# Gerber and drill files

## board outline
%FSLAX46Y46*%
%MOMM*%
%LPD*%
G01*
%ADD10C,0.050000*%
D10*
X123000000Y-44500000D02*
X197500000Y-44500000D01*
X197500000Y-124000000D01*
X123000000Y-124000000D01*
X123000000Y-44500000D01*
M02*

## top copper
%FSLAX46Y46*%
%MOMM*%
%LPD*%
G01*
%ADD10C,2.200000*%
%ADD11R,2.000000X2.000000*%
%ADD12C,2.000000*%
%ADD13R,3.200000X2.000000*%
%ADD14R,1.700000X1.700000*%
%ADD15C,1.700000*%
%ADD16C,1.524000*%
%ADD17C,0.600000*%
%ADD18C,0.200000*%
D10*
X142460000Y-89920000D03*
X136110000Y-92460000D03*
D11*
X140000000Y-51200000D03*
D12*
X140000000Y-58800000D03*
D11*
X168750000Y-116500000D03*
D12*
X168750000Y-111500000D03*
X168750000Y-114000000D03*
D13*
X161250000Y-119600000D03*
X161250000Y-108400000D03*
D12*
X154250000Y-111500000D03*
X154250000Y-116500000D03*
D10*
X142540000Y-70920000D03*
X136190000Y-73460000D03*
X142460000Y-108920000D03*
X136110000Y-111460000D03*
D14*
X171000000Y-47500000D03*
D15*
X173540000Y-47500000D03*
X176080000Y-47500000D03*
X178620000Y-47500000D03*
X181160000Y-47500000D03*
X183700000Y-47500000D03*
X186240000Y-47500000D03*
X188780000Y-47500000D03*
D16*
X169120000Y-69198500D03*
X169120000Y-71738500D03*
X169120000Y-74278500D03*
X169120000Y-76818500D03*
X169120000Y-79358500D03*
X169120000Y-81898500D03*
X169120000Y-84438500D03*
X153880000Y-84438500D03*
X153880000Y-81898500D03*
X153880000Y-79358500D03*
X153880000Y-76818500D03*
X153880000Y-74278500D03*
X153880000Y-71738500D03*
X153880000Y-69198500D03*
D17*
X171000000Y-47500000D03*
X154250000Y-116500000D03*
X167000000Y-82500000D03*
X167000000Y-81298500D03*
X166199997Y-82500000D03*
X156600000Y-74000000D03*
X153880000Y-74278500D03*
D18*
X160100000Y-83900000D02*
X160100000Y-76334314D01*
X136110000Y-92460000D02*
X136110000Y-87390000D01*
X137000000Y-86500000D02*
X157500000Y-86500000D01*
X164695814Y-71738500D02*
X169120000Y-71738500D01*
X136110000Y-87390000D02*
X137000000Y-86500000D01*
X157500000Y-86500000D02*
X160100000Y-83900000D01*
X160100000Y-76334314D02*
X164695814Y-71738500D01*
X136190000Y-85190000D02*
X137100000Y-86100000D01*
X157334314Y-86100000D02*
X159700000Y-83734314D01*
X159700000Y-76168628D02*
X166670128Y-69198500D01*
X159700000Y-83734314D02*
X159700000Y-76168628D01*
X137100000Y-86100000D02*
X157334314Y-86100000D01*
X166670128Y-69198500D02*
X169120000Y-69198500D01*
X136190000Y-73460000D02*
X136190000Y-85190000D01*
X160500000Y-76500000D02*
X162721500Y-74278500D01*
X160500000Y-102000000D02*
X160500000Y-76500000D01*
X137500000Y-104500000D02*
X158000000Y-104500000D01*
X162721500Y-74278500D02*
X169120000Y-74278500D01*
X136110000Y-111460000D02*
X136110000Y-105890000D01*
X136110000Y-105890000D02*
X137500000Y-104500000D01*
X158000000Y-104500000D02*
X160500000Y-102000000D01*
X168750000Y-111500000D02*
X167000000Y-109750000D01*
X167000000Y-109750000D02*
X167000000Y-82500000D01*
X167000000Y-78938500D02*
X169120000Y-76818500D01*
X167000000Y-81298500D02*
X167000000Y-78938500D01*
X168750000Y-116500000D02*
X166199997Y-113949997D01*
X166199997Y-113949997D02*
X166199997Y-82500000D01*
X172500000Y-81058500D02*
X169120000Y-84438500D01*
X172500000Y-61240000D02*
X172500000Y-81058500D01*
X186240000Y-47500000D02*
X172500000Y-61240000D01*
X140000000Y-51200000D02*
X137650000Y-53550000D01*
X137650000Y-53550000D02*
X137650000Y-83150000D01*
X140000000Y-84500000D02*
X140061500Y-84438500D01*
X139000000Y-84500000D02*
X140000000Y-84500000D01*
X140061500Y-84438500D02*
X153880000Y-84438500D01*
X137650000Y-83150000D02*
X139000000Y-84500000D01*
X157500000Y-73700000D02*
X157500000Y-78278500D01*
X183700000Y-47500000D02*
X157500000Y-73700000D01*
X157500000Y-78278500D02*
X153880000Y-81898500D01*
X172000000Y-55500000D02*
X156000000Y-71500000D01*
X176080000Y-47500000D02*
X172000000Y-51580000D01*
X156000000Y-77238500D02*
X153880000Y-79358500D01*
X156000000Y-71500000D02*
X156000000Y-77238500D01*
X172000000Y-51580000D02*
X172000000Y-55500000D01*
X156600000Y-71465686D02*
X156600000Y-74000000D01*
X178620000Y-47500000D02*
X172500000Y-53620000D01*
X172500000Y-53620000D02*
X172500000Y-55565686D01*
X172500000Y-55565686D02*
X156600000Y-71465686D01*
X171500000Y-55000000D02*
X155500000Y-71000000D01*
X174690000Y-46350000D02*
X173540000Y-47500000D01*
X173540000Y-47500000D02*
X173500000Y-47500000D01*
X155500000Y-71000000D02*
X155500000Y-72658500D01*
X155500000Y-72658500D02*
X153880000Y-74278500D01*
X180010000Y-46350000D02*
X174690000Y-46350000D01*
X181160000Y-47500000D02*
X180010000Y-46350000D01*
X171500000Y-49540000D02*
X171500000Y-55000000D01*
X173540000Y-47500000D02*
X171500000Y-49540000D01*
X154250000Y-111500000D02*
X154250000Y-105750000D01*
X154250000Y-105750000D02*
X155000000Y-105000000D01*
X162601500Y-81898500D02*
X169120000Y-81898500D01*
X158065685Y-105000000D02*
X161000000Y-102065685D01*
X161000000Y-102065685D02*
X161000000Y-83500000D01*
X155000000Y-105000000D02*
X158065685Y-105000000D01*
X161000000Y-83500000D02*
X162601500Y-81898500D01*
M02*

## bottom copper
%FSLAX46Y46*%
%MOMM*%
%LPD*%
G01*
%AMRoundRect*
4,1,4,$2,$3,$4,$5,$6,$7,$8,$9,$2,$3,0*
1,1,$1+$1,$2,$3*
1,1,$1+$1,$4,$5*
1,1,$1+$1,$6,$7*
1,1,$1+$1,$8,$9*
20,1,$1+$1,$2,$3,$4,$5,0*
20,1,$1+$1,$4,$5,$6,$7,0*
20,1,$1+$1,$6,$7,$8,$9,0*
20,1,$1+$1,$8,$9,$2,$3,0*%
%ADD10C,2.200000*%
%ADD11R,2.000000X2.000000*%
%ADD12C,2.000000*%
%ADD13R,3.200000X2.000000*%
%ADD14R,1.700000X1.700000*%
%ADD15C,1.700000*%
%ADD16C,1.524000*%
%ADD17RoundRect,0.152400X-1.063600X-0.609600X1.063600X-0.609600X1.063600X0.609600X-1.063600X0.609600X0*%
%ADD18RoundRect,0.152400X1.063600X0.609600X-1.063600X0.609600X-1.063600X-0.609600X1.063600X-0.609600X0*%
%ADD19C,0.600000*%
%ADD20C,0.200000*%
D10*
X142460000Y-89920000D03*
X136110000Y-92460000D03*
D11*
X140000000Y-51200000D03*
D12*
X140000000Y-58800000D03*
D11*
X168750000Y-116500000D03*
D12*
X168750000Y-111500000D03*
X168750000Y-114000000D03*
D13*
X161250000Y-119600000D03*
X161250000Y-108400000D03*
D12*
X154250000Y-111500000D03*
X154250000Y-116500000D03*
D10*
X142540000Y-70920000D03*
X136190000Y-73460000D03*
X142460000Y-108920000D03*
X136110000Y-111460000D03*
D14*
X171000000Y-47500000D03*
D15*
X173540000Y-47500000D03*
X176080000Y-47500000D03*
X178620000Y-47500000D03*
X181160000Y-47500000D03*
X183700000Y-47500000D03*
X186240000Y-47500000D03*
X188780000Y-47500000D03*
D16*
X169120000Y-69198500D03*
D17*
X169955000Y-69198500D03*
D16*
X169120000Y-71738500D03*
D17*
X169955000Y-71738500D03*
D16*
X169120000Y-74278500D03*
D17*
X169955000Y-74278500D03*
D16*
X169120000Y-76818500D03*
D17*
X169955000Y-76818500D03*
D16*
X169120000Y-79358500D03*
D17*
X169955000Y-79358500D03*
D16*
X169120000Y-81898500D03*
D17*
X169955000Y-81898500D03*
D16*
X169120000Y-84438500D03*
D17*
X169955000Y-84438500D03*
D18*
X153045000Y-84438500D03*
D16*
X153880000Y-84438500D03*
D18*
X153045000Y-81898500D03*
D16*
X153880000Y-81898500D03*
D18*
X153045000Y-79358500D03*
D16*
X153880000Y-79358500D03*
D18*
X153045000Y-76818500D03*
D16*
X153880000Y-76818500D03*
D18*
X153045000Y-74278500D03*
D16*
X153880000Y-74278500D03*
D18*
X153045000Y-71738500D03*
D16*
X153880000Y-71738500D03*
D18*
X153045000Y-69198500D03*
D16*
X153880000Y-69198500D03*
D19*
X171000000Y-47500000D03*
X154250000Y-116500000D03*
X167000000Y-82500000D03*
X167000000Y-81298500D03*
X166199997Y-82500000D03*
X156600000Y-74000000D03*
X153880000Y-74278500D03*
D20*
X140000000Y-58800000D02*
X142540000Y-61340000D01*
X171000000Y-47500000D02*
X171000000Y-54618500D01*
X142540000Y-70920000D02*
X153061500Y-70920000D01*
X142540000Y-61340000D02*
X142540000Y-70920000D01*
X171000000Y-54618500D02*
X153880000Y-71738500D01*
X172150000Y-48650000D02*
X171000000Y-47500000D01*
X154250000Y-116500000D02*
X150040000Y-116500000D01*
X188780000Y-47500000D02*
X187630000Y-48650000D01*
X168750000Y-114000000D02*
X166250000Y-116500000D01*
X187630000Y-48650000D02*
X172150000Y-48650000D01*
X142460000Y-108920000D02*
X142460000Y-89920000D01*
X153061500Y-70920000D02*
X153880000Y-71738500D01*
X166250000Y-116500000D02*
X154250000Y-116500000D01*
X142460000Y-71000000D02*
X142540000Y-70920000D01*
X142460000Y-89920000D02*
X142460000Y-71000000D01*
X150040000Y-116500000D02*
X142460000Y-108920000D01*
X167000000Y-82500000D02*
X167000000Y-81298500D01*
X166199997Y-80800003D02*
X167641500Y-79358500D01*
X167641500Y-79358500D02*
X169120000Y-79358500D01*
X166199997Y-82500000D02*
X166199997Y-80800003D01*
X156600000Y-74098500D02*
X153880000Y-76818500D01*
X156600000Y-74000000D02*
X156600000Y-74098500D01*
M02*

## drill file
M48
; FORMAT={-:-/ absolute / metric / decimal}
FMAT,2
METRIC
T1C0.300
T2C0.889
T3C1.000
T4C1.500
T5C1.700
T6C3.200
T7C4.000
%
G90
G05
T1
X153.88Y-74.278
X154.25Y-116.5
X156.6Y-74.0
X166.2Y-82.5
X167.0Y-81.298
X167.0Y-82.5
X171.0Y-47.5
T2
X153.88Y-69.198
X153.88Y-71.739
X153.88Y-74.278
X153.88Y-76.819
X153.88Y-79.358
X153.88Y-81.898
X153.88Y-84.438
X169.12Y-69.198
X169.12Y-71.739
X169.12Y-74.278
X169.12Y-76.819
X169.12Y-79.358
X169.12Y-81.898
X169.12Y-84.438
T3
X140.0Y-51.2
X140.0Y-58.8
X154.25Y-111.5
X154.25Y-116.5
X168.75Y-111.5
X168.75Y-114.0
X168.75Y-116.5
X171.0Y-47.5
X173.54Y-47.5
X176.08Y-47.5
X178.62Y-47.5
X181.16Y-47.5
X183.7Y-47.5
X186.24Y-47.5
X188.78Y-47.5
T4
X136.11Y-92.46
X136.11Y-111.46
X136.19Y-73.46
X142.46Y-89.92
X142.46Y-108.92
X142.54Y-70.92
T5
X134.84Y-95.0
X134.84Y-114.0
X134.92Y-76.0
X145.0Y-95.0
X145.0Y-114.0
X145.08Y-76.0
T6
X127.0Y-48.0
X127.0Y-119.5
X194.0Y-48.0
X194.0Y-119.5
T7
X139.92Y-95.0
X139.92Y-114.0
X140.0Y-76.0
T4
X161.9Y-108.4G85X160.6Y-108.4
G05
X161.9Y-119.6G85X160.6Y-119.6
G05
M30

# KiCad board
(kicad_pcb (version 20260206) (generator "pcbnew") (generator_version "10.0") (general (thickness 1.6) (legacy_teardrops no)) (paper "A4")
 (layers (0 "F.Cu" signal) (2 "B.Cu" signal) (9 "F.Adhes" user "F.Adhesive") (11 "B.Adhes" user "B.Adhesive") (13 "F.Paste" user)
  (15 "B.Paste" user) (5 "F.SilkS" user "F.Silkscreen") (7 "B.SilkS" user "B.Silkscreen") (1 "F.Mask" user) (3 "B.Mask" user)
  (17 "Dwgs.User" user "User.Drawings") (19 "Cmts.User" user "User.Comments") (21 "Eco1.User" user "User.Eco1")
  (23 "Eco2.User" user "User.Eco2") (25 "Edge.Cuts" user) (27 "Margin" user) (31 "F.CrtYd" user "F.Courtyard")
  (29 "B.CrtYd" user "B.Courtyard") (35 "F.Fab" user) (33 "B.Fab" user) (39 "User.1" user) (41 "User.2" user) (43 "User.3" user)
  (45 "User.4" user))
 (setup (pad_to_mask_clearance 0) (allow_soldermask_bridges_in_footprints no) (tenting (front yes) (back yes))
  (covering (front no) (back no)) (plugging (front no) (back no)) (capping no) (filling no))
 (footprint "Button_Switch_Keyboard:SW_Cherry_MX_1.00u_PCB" (layer "F.Cu") (at 142.46 89.92)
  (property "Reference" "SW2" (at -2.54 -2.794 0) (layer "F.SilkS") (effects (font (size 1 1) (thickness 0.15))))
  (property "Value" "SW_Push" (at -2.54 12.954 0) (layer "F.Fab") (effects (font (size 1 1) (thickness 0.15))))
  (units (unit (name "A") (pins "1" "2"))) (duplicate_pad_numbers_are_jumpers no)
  (pad "" np_thru_hole circle (at -7.62 5.08) (size 1.7 1.7) (drill 1.7) (layers "*.Cu" "*.Mask"))
  (pad "" np_thru_hole circle (at -2.54 5.08) (size 4 4) (drill 4) (layers "*.Cu" "*.Mask"))
  (pad "" np_thru_hole circle (at 2.54 5.08) (size 1.7 1.7) (drill 1.7) (layers "*.Cu" "*.Mask"))
  (pad "1" thru_hole circle (at 0 0) (size 2.2 2.2) (drill 1.5) (layers "*.Cu" "*.Mask") (remove_unused_layers no) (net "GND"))
  (pad "2" thru_hole circle (at -6.35 2.54) (size 2.2 2.2) (drill 1.5) (layers "*.Cu" "*.Mask") (remove_unused_layers no)
   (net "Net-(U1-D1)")))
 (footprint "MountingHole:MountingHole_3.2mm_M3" (layer "F.Cu") (at 194 48 180)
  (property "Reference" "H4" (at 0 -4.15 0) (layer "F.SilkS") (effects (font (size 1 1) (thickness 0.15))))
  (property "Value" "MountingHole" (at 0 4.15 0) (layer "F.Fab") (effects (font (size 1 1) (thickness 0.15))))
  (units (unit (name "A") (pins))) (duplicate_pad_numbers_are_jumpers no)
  (pad "" np_thru_hole circle (at 0 0 180) (size 3.2 3.2) (drill 3.2) (layers "*.Cu" "*.Mask")))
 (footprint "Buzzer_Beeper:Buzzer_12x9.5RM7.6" (layer "F.Cu") (at 140 51.2 -90)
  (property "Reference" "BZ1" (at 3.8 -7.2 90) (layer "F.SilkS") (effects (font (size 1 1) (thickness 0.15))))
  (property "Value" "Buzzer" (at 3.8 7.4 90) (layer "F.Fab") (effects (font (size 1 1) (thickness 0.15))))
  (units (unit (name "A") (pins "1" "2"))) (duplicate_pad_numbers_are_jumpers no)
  (pad "1" thru_hole rect (at 0 0 270) (size 2 2) (drill 1) (layers "*.Cu" "*.Mask") (remove_unused_layers no) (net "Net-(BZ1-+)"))
  (pad "2" thru_hole circle (at 7.6 0 270) (size 2 2) (drill 1) (layers "*.Cu" "*.Mask") (remove_unused_layers no) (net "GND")))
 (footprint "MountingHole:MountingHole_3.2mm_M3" (layer "F.Cu") (at 127 48 180)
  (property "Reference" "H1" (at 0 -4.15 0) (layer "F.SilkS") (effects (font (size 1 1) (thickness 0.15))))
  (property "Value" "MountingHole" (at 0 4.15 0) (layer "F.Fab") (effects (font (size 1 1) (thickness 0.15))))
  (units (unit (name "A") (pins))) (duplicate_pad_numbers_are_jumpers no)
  (pad "" np_thru_hole circle (at 0 0 180) (size 3.2 3.2) (drill 3.2) (layers "*.Cu" "*.Mask")))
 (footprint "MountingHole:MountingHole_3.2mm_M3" (layer "F.Cu") (at 127 119.5 180)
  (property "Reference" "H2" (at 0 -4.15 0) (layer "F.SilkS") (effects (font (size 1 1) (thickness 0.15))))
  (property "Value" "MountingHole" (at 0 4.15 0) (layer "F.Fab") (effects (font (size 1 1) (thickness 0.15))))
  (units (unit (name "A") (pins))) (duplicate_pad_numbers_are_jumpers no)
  (pad "" np_thru_hole circle (at 0 0 180) (size 3.2 3.2) (drill 3.2) (layers "*.Cu" "*.Mask")))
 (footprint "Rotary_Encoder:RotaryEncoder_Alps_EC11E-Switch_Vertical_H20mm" (layer "F.Cu") (at 168.75 116.5 180)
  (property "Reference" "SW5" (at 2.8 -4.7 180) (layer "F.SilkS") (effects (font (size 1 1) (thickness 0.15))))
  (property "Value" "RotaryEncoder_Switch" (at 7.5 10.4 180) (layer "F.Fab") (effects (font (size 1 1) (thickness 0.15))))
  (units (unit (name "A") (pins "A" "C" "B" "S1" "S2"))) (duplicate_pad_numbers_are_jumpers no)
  (pad "A" thru_hole rect (at 0 0 180) (size 2 2) (drill 1) (layers "*.Cu" "*.Mask") (remove_unused_layers no) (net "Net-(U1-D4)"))
  (pad "B" thru_hole circle (at 0 5 180) (size 2 2) (drill 1) (layers "*.Cu" "*.Mask") (remove_unused_layers no) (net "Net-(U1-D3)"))
  (pad "C" thru_hole circle (at 0 2.5 180) (size 2 2) (drill 1) (layers "*.Cu" "*.Mask") (remove_unused_layers no) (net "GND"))
  (pad "MP" thru_hole rect (at 7.5 -3.1 180) (size 3.2 2) (drill oval 2.8 1.5) (layers "*.Cu" "*.Mask") (remove_unused_layers no))
  (pad "MP" thru_hole rect (at 7.5 8.1 180) (size 3.2 2) (drill oval 2.8 1.5) (layers "*.Cu" "*.Mask") (remove_unused_layers no))
  (pad "S1" thru_hole circle (at 14.5 5 180) (size 2 2) (drill 1) (layers "*.Cu" "*.Mask") (remove_unused_layers no) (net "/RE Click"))
  (pad "S2" thru_hole circle (at 14.5 0 180) (size 2 2) (drill 1) (layers "*.Cu" "*.Mask") (remove_unused_layers no) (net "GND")))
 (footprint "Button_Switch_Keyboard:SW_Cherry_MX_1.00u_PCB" (layer "F.Cu") (at 142.54 70.92)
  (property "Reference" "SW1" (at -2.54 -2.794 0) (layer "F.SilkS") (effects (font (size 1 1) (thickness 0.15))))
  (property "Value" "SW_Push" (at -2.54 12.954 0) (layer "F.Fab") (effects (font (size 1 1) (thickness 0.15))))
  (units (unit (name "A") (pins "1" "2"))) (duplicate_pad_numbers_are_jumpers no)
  (pad "" np_thru_hole circle (at -7.62 5.08) (size 1.7 1.7) (drill 1.7) (layers "*.Cu" "*.Mask"))
  (pad "" np_thru_hole circle (at -2.54 5.08) (size 4 4) (drill 4) (layers "*.Cu" "*.Mask"))
  (pad "" np_thru_hole circle (at 2.54 5.08) (size 1.7 1.7) (drill 1.7) (layers "*.Cu" "*.Mask"))
  (pad "1" thru_hole circle (at 0 0) (size 2.2 2.2) (drill 1.5) (layers "*.Cu" "*.Mask") (remove_unused_layers no) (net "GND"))
  (pad "2" thru_hole circle (at -6.35 2.54) (size 2.2 2.2) (drill 1.5) (layers "*.Cu" "*.Mask") (remove_unused_layers no)
   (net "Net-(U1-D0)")))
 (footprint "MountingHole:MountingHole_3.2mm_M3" (layer "F.Cu") (at 194 119.5 180)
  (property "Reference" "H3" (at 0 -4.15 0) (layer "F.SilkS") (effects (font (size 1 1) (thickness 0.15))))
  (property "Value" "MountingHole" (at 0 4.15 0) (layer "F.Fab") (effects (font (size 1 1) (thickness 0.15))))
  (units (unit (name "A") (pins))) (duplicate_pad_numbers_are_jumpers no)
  (pad "" np_thru_hole circle (at 0 0 180) (size 3.2 3.2) (drill 3.2) (layers "*.Cu" "*.Mask")))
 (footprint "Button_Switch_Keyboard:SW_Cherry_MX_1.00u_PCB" (layer "F.Cu") (at 142.46 108.92)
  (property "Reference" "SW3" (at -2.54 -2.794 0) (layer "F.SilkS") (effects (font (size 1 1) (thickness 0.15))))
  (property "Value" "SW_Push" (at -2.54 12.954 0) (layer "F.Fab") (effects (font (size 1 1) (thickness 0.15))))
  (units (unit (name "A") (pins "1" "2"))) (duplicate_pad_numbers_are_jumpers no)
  (pad "" np_thru_hole circle (at -7.62 5.08) (size 1.7 1.7) (drill 1.7) (layers "*.Cu" "*.Mask"))
  (pad "" np_thru_hole circle (at -2.54 5.08) (size 4 4) (drill 4) (layers "*.Cu" "*.Mask"))
  (pad "" np_thru_hole circle (at 2.54 5.08) (size 1.7 1.7) (drill 1.7) (layers "*.Cu" "*.Mask"))
  (pad "1" thru_hole circle (at 0 0) (size 2.2 2.2) (drill 1.5) (layers "*.Cu" "*.Mask") (remove_unused_layers no) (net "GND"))
  (pad "2" thru_hole circle (at -6.35 2.54) (size 2.2 2.2) (drill 1.5) (layers "*.Cu" "*.Mask") (remove_unused_layers no)
   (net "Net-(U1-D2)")))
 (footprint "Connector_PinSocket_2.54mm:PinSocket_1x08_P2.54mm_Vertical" (layer "F.Cu") (at 171 47.5 90)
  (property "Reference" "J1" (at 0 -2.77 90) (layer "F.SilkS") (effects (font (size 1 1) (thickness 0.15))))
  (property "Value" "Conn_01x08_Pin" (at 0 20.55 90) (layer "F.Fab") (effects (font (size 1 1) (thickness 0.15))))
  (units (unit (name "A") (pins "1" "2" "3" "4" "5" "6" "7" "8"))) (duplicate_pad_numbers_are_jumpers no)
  (pad "1" thru_hole rect (at 0 0 90) (size 1.7 1.7) (drill 1) (layers "*.Cu" "*.Mask") (remove_unused_layers no) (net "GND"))
  (pad "2" thru_hole circle (at 0 2.54 90) (size 1.7 1.7) (drill 1) (layers "*.Cu" "*.Mask") (remove_unused_layers no) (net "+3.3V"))
  (pad "3" thru_hole circle (at 0 5.08 90) (size 1.7 1.7) (drill 1) (layers "*.Cu" "*.Mask") (remove_unused_layers no) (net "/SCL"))
  (pad "4" thru_hole circle (at 0 7.62 90) (size 1.7 1.7) (drill 1) (layers "*.Cu" "*.Mask") (remove_unused_layers no) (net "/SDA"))
  (pad "5" thru_hole circle (at 0 10.16 90) (size 1.7 1.7) (drill 1) (layers "*.Cu" "*.Mask") (remove_unused_layers no) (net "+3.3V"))
  (pad "6" thru_hole circle (at 0 12.7 90) (size 1.7 1.7) (drill 1) (layers "*.Cu" "*.Mask") (remove_unused_layers no) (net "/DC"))
  (pad "7" thru_hole circle (at 0 15.24 90) (size 1.7 1.7) (drill 1) (layers "*.Cu" "*.Mask") (remove_unused_layers no) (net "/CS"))
  (pad "8" thru_hole circle (at 0 17.78 90) (size 1.7 1.7) (drill 1) (layers "*.Cu" "*.Mask") (remove_unused_layers no) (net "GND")))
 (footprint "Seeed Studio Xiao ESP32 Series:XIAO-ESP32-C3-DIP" (layer "B.Cu") (at 161.5 76.8185 90)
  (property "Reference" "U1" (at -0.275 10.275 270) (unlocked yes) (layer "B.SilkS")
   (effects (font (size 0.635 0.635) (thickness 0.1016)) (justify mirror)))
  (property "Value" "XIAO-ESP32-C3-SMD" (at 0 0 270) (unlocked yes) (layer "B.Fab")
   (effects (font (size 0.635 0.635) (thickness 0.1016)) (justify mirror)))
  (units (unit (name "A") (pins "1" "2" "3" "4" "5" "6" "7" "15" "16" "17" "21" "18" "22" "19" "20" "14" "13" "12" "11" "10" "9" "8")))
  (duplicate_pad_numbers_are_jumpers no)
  (pad "1" thru_hole circle (at 7.62 7.62) (size 1.524 1.524) (drill 0.889) (layers "*.Cu" "*.Mask") (remove_unused_layers no)
   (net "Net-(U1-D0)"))
  (pad "1" smd roundrect (at 7.62 8.455) (size 2.432 1.524) (layers "B.Cu" "B.Mask") (roundrect_rratio 0.1) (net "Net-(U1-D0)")
   (thermal_bridge_angle 45))
  (pad "2" thru_hole circle (at 5.08 7.62) (size 1.524 1.524) (drill 0.889) (layers "*.Cu" "*.Mask") (remove_unused_layers no)
   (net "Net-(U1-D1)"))
  (pad "2" smd roundrect (at 5.08 8.455) (size 2.432 1.524) (layers "B.Cu" "B.Mask") (roundrect_rratio 0.1) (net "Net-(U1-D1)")
   (thermal_bridge_angle 45))
  (pad "3" thru_hole circle (at 2.54 7.62) (size 1.524 1.524) (drill 0.889) (layers "*.Cu" "*.Mask") (remove_unused_layers no)
   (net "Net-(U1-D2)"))
  (pad "3" smd roundrect (at 2.54 8.455) (size 2.432 1.524) (layers "B.Cu" "B.Mask") (roundrect_rratio 0.1) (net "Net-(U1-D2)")
   (thermal_bridge_angle 45))
  (pad "4" thru_hole circle (at 0 7.62) (size 1.524 1.524) (drill 0.889) (layers "*.Cu" "*.Mask") (remove_unused_layers no)
   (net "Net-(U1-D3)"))
  (pad "4" smd roundrect (at 0 8.455) (size 2.432 1.524) (layers "B.Cu" "B.Mask") (roundrect_rratio 0.1) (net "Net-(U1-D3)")
   (thermal_bridge_angle 45))
  (pad "5" thru_hole circle (at -2.54 7.62) (size 1.524 1.524) (drill 0.889) (layers "*.Cu" "*.Mask") (remove_unused_layers no)
   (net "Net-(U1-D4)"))
  (pad "5" smd roundrect (at -2.54 8.455) (size 2.432 1.524) (layers "B.Cu" "B.Mask") (roundrect_rratio 0.1) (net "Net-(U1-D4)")
   (thermal_bridge_angle 45))
  (pad "6" thru_hole circle (at -5.08 7.62) (size 1.524 1.524) (drill 0.889) (layers "*.Cu" "*.Mask") (remove_unused_layers no)
   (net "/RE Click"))
  (pad "6" smd roundrect (at -5.08 8.455) (size 2.432 1.524) (layers "B.Cu" "B.Mask") (roundrect_rratio 0.1) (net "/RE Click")
   (thermal_bridge_angle 45))
  (pad "7" thru_hole circle (at -7.62 7.62) (size 1.524 1.524) (drill 0.889) (layers "*.Cu" "*.Mask") (remove_unused_layers no) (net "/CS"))
  (pad "7" smd roundrect (at -7.62 8.455) (size 2.432 1.524) (layers "B.Cu" "B.Mask") (roundrect_rratio 0.1) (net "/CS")
   (thermal_bridge_angle 45))
  (pad "8" smd roundrect (at -7.62 -8.455 180) (size 2.432 1.524) (layers "B.Cu" "B.Mask") (roundrect_rratio 0.1) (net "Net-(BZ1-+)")
   (thermal_bridge_angle 45))
  (pad "8" thru_hole circle (at -7.62 -7.62 180) (size 1.524 1.524) (drill 0.889) (layers "*.Cu" "*.Mask") (remove_unused_layers no)
   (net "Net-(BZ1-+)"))
  (pad "9" smd roundrect (at -5.08 -8.455 180) (size 2.432 1.524) (layers "B.Cu" "B.Mask") (roundrect_rratio 0.1) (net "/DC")
   (thermal_bridge_angle 45))
  (pad "9" thru_hole circle (at -5.08 -7.62 180) (size 1.524 1.524) (drill 0.889) (layers "*.Cu" "*.Mask") (remove_unused_layers no)
   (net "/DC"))
  (pad "10" smd roundrect (at -2.54 -8.455 180) (size 2.432 1.524) (layers "B.Cu" "B.Mask") (roundrect_rratio 0.1) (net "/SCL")
   (thermal_bridge_angle 45))
  (pad "10" thru_hole circle (at -2.54 -7.62 180) (size 1.524 1.524) (drill 0.889) (layers "*.Cu" "*.Mask") (remove_unused_layers no)
   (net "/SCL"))
  (pad "11" smd roundrect (at 0 -8.455 180) (size 2.432 1.524) (layers "B.Cu" "B.Mask") (roundrect_rratio 0.1) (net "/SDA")
   (thermal_bridge_angle 45))
  (pad "11" thru_hole circle (at 0 -7.62 180) (size 1.524 1.524) (drill 0.889) (layers "*.Cu" "*.Mask") (remove_unused_layers no)
   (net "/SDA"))
  (pad "12" smd roundrect (at 2.54 -8.455 180) (size 2.432 1.524) (layers "B.Cu" "B.Mask") (roundrect_rratio 0.1) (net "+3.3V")
   (thermal_bridge_angle 45))
  (pad "12" thru_hole circle (at 2.54 -7.62 180) (size 1.524 1.524) (drill 0.889) (layers "*.Cu" "*.Mask") (remove_unused_layers no)
   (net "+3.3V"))
  (pad "13" smd roundrect (at 5.08 -8.455 180) (size 2.432 1.524) (layers "B.Cu" "B.Mask") (roundrect_rratio 0.1) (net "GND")
   (thermal_bridge_angle 45))
  (pad "13" thru_hole circle (at 5.08 -7.62 180) (size 1.524 1.524) (drill 0.889) (layers "*.Cu" "*.Mask") (remove_unused_layers no)
   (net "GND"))
  (pad "14" smd roundrect (at 7.62 -8.455 180) (size 2.432 1.524) (layers "B.Cu" "B.Mask") (roundrect_rratio 0.1)
   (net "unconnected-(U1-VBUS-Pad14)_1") (thermal_bridge_angle 45))
  (pad "14" thru_hole circle (at 7.62 -7.62 180) (size 1.524 1.524) (drill 0.889) (layers "*.Cu" "*.Mask") (remove_unused_layers no)
   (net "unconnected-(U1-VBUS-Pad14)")))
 (gr_rect (start 123 44.5) (end 197.5 124) (stroke (width 0.05) (type default)) (fill no) (layer "Edge.Cuts"))
 (via (at 171 47.5) (size 0.6) (drill 0.3) (layers "F.Cu" "B.Cu") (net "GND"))
 (via (at 154.25 116.5) (size 0.6) (drill 0.3) (layers "F.Cu" "B.Cu") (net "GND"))
 (segment (start 140 58.8) (end 142.54 61.34) (width 0.2) (layer "B.Cu") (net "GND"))
 (segment (start 171 47.5) (end 171 54.6185) (width 0.2) (layer "B.Cu") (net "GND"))
 (segment (start 142.54 70.92) (end 153.0615 70.92) (width 0.2) (layer "B.Cu") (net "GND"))
 (segment (start 142.54 61.34) (end 142.54 70.92) (width 0.2) (layer "B.Cu") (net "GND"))
 (segment (start 171 54.6185) (end 153.88 71.7385) (width 0.2) (layer "B.Cu") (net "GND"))
 (segment (start 172.15 48.65) (end 171 47.5) (width 0.2) (layer "B.Cu") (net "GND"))
 (segment (start 154.25 116.5) (end 150.04 116.5) (width 0.2) (layer "B.Cu") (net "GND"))
 (segment (start 188.78 47.5) (end 187.63 48.65) (width 0.2) (layer "B.Cu") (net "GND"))
 (segment (start 168.75 114) (end 166.25 116.5) (width 0.2) (layer "B.Cu") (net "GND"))
 (segment (start 187.63 48.65) (end 172.15 48.65) (width 0.2) (layer "B.Cu") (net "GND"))
 (segment (start 142.46 108.92) (end 142.46 89.92) (width 0.2) (layer "B.Cu") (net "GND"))
 (segment (start 153.0615 70.92) (end 153.88 71.7385) (width 0.2) (layer "B.Cu") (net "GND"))
 (segment (start 166.25 116.5) (end 154.25 116.5) (width 0.2) (layer "B.Cu") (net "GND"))
 (segment (start 142.46 71) (end 142.54 70.92) (width 0.2) (layer "B.Cu") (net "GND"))
 (segment (start 142.46 89.92) (end 142.46 71) (width 0.2) (layer "B.Cu") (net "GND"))
 (segment (start 150.04 116.5) (end 142.46 108.92) (width 0.2) (layer "B.Cu") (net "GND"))
 (segment (start 160.1 83.9) (end 160.1 76.334314) (width 0.2) (layer "F.Cu") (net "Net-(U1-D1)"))
 (segment (start 136.11 92.46) (end 136.11 87.39) (width 0.2) (layer "F.Cu") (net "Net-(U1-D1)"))
 (segment (start 137 86.5) (end 157.5 86.5) (width 0.2) (layer "F.Cu") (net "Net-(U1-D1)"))
 (segment (start 164.695814 71.7385) (end 169.12 71.7385) (width 0.2) (layer "F.Cu") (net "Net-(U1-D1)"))
 (segment (start 136.11 87.39) (end 137 86.5) (width 0.2) (layer "F.Cu") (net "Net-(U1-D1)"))
 (segment (start 157.5 86.5) (end 160.1 83.9) (width 0.2) (layer "F.Cu") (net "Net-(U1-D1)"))
 (segment (start 160.1 76.334314) (end 164.695814 71.7385) (width 0.2) (layer "F.Cu") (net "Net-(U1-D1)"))
 (segment (start 136.19 85.19) (end 137.1 86.1) (width 0.2) (layer "F.Cu") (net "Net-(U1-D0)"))
 (segment (start 157.334314 86.1) (end 159.7 83.734314) (width 0.2) (layer "F.Cu") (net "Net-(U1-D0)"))
 (segment (start 159.7 76.168628) (end 166.670128 69.1985) (width 0.2) (layer "F.Cu") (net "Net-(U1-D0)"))
 (segment (start 159.7 83.734314) (end 159.7 76.168628) (width 0.2) (layer "F.Cu") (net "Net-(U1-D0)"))
 (segment (start 137.1 86.1) (end 157.334314 86.1) (width 0.2) (layer "F.Cu") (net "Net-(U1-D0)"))
 (segment (start 166.670128 69.1985) (end 169.12 69.1985) (width 0.2) (layer "F.Cu") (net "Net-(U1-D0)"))
 (segment (start 136.19 73.46) (end 136.19 85.19) (width 0.2) (layer "F.Cu") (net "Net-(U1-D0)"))
 (segment (start 160.5 76.5) (end 162.7215 74.2785) (width 0.2) (layer "F.Cu") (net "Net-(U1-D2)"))
 (segment (start 160.5 102) (end 160.5 76.5) (width 0.2) (layer "F.Cu") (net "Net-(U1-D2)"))
 (segment (start 137.5 104.5) (end 158 104.5) (width 0.2) (layer "F.Cu") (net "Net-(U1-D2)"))
 (segment (start 162.7215 74.2785) (end 169.12 74.2785) (width 0.2) (layer "F.Cu") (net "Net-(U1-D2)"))
 (segment (start 136.11 111.46) (end 136.11 105.89) (width 0.2) (layer "F.Cu") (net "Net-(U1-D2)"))
 (segment (start 136.11 105.89) (end 137.5 104.5) (width 0.2) (layer "F.Cu") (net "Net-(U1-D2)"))
 (segment (start 158 104.5) (end 160.5 102) (width 0.2) (layer "F.Cu") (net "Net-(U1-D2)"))
 (segment (start 168.75 111.5) (end 167 109.75) (width 0.2) (layer "F.Cu") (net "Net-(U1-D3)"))
 (segment (start 167 109.75) (end 167 82.5) (width 0.2) (layer "F.Cu") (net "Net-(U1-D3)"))
 (segment (start 167 78.9385) (end 169.12 76.8185) (width 0.2) (layer "F.Cu") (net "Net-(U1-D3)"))
 (segment (start 167 81.2985) (end 167 78.9385) (width 0.2) (layer "F.Cu") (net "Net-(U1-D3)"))
 (via (at 167 82.5) (size 0.6) (drill 0.3) (layers "F.Cu" "B.Cu") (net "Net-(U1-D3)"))
 (via (at 167 81.2985) (size 0.6) (drill 0.3) (layers "F.Cu" "B.Cu") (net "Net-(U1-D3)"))
 (segment (start 167 82.5) (end 167 81.2985) (width 0.2) (layer "B.Cu") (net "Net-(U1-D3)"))
 (segment (start 168.75 116.5) (end 166.199997 113.949997) (width 0.2) (layer "F.Cu") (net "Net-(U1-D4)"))
 (segment (start 166.199997 113.949997) (end 166.199997 82.5) (width 0.2) (layer "F.Cu") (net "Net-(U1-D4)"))
 (via (at 166.199997 82.5) (size 0.6) (drill 0.3) (layers "F.Cu" "B.Cu") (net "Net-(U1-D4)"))
 (segment (start 166.199997 80.800003) (end 167.6415 79.3585) (width 0.2) (layer "B.Cu") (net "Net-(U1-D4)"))
 (segment (start 167.6415 79.3585) (end 169.12 79.3585) (width 0.2) (layer "B.Cu") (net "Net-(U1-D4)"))
 (segment (start 166.199997 82.5) (end 166.199997 80.800003) (width 0.2) (layer "B.Cu") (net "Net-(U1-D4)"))
 (segment (start 172.5 81.0585) (end 169.12 84.4385) (width 0.2) (layer "F.Cu") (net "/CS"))
 (segment (start 172.5 61.24) (end 172.5 81.0585) (width 0.2) (layer "F.Cu") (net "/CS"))
 (segment (start 186.24 47.5) (end 172.5 61.24) (width 0.2) (layer "F.Cu") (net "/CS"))
 (segment (start 140 51.2) (end 137.65 53.55) (width 0.2) (layer "F.Cu") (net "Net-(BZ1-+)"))
 (segment (start 137.65 53.55) (end 137.65 83.15) (width 0.2) (layer "F.Cu") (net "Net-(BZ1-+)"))
 (segment (start 140 84.5) (end 140.0615 84.4385) (width 0.2) (layer "F.Cu") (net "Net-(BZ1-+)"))
 (segment (start 139 84.5) (end 140 84.5) (width 0.2) (layer "F.Cu") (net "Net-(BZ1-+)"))
 (segment (start 140.0615 84.4385) (end 153.88 84.4385) (width 0.2) (layer "F.Cu") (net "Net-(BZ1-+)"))
 (segment (start 137.65 83.15) (end 139 84.5) (width 0.2) (layer "F.Cu") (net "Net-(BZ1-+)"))
 (segment (start 157.5 73.7) (end 157.5 78.2785) (width 0.2) (layer "F.Cu") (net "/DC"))
 (segment (start 183.7 47.5) (end 157.5 73.7) (width 0.2) (layer "F.Cu") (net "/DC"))
 (segment (start 157.5 78.2785) (end 153.88 81.8985) (width 0.2) (layer "F.Cu") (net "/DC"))
 (segment (start 172 55.5) (end 156 71.5) (width 0.2) (layer "F.Cu") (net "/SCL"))
 (segment (start 176.08 47.5) (end 172 51.58) (width 0.2) (layer "F.Cu") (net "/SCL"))
 (segment (start 156 77.2385) (end 153.88 79.3585) (width 0.2) (layer "F.Cu") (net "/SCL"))
 (segment (start 156 71.5) (end 156 77.2385) (width 0.2) (layer "F.Cu") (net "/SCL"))
 (segment (start 172 51.58) (end 172 55.5) (width 0.2) (layer "F.Cu") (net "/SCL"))
 (segment (start 156.6 71.465686) (end 156.6 74) (width 0.2) (layer "F.Cu") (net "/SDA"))
 (segment (start 178.62 47.5) (end 172.5 53.62) (width 0.2) (layer "F.Cu") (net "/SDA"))
 (segment (start 172.5 53.62) (end 172.5 55.565686) (width 0.2) (layer "F.Cu") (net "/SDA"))
 (segment (start 172.5 55.565686) (end 156.6 71.465686) (width 0.2) (layer "F.Cu") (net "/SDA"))
 (via (at 156.6 74) (size 0.6) (drill 0.3) (layers "F.Cu" "B.Cu") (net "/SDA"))
 (segment (start 156.6 74.0985) (end 153.88 76.8185) (width 0.2) (layer "B.Cu") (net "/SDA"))
 (segment (start 156.6 74) (end 156.6 74.0985) (width 0.2) (layer "B.Cu") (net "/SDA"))
 (segment (start 171.5 55) (end 155.5 71) (width 0.2) (layer "F.Cu") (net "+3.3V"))
 (segment (start 174.69 46.35) (end 173.54 47.5) (width 0.2) (layer "F.Cu") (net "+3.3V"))
 (segment (start 173.54 47.5) (end 173.5 47.5) (width 0.2) (layer "F.Cu") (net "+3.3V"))
 (segment (start 155.5 71) (end 155.5 72.6585) (width 0.2) (layer "F.Cu") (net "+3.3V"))
 (segment (start 155.5 72.6585) (end 153.88 74.2785) (width 0.2) (layer "F.Cu") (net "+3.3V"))
 (segment (start 180.01 46.35) (end 174.69 46.35) (width 0.2) (layer "F.Cu") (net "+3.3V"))
 (segment (start 181.16 47.5) (end 180.01 46.35) (width 0.2) (layer "F.Cu") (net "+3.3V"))
 (segment (start 171.5 49.54) (end 171.5 55) (width 0.2) (layer "F.Cu") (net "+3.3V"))
 (segment (start 173.54 47.5) (end 171.5 49.54) (width 0.2) (layer "F.Cu") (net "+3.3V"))
 (via (at 153.88 74.2785) (size 0.6) (drill 0.3) (layers "F.Cu" "B.Cu") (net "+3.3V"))
 (segment (start 154.25 111.5) (end 154.25 105.75) (width 0.2) (layer "F.Cu") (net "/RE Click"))
 (segment (start 154.25 105.75) (end 155 105) (width 0.2) (layer "F.Cu") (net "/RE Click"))
 (segment (start 162.6015 81.8985) (end 169.12 81.8985) (width 0.2) (layer "F.Cu") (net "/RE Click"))
 (segment (start 158.065685 105) (end 161 102.065685) (width 0.2) (layer "F.Cu") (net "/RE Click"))
 (segment (start 161 102.065685) (end 161 83.5) (width 0.2) (layer "F.Cu") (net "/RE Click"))
 (segment (start 155 105) (end 158.065685 105) (width 0.2) (layer "F.Cu") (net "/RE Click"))
 (segment (start 161 83.5) (end 162.6015 81.8985) (width 0.2) (layer "F.Cu") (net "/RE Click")))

